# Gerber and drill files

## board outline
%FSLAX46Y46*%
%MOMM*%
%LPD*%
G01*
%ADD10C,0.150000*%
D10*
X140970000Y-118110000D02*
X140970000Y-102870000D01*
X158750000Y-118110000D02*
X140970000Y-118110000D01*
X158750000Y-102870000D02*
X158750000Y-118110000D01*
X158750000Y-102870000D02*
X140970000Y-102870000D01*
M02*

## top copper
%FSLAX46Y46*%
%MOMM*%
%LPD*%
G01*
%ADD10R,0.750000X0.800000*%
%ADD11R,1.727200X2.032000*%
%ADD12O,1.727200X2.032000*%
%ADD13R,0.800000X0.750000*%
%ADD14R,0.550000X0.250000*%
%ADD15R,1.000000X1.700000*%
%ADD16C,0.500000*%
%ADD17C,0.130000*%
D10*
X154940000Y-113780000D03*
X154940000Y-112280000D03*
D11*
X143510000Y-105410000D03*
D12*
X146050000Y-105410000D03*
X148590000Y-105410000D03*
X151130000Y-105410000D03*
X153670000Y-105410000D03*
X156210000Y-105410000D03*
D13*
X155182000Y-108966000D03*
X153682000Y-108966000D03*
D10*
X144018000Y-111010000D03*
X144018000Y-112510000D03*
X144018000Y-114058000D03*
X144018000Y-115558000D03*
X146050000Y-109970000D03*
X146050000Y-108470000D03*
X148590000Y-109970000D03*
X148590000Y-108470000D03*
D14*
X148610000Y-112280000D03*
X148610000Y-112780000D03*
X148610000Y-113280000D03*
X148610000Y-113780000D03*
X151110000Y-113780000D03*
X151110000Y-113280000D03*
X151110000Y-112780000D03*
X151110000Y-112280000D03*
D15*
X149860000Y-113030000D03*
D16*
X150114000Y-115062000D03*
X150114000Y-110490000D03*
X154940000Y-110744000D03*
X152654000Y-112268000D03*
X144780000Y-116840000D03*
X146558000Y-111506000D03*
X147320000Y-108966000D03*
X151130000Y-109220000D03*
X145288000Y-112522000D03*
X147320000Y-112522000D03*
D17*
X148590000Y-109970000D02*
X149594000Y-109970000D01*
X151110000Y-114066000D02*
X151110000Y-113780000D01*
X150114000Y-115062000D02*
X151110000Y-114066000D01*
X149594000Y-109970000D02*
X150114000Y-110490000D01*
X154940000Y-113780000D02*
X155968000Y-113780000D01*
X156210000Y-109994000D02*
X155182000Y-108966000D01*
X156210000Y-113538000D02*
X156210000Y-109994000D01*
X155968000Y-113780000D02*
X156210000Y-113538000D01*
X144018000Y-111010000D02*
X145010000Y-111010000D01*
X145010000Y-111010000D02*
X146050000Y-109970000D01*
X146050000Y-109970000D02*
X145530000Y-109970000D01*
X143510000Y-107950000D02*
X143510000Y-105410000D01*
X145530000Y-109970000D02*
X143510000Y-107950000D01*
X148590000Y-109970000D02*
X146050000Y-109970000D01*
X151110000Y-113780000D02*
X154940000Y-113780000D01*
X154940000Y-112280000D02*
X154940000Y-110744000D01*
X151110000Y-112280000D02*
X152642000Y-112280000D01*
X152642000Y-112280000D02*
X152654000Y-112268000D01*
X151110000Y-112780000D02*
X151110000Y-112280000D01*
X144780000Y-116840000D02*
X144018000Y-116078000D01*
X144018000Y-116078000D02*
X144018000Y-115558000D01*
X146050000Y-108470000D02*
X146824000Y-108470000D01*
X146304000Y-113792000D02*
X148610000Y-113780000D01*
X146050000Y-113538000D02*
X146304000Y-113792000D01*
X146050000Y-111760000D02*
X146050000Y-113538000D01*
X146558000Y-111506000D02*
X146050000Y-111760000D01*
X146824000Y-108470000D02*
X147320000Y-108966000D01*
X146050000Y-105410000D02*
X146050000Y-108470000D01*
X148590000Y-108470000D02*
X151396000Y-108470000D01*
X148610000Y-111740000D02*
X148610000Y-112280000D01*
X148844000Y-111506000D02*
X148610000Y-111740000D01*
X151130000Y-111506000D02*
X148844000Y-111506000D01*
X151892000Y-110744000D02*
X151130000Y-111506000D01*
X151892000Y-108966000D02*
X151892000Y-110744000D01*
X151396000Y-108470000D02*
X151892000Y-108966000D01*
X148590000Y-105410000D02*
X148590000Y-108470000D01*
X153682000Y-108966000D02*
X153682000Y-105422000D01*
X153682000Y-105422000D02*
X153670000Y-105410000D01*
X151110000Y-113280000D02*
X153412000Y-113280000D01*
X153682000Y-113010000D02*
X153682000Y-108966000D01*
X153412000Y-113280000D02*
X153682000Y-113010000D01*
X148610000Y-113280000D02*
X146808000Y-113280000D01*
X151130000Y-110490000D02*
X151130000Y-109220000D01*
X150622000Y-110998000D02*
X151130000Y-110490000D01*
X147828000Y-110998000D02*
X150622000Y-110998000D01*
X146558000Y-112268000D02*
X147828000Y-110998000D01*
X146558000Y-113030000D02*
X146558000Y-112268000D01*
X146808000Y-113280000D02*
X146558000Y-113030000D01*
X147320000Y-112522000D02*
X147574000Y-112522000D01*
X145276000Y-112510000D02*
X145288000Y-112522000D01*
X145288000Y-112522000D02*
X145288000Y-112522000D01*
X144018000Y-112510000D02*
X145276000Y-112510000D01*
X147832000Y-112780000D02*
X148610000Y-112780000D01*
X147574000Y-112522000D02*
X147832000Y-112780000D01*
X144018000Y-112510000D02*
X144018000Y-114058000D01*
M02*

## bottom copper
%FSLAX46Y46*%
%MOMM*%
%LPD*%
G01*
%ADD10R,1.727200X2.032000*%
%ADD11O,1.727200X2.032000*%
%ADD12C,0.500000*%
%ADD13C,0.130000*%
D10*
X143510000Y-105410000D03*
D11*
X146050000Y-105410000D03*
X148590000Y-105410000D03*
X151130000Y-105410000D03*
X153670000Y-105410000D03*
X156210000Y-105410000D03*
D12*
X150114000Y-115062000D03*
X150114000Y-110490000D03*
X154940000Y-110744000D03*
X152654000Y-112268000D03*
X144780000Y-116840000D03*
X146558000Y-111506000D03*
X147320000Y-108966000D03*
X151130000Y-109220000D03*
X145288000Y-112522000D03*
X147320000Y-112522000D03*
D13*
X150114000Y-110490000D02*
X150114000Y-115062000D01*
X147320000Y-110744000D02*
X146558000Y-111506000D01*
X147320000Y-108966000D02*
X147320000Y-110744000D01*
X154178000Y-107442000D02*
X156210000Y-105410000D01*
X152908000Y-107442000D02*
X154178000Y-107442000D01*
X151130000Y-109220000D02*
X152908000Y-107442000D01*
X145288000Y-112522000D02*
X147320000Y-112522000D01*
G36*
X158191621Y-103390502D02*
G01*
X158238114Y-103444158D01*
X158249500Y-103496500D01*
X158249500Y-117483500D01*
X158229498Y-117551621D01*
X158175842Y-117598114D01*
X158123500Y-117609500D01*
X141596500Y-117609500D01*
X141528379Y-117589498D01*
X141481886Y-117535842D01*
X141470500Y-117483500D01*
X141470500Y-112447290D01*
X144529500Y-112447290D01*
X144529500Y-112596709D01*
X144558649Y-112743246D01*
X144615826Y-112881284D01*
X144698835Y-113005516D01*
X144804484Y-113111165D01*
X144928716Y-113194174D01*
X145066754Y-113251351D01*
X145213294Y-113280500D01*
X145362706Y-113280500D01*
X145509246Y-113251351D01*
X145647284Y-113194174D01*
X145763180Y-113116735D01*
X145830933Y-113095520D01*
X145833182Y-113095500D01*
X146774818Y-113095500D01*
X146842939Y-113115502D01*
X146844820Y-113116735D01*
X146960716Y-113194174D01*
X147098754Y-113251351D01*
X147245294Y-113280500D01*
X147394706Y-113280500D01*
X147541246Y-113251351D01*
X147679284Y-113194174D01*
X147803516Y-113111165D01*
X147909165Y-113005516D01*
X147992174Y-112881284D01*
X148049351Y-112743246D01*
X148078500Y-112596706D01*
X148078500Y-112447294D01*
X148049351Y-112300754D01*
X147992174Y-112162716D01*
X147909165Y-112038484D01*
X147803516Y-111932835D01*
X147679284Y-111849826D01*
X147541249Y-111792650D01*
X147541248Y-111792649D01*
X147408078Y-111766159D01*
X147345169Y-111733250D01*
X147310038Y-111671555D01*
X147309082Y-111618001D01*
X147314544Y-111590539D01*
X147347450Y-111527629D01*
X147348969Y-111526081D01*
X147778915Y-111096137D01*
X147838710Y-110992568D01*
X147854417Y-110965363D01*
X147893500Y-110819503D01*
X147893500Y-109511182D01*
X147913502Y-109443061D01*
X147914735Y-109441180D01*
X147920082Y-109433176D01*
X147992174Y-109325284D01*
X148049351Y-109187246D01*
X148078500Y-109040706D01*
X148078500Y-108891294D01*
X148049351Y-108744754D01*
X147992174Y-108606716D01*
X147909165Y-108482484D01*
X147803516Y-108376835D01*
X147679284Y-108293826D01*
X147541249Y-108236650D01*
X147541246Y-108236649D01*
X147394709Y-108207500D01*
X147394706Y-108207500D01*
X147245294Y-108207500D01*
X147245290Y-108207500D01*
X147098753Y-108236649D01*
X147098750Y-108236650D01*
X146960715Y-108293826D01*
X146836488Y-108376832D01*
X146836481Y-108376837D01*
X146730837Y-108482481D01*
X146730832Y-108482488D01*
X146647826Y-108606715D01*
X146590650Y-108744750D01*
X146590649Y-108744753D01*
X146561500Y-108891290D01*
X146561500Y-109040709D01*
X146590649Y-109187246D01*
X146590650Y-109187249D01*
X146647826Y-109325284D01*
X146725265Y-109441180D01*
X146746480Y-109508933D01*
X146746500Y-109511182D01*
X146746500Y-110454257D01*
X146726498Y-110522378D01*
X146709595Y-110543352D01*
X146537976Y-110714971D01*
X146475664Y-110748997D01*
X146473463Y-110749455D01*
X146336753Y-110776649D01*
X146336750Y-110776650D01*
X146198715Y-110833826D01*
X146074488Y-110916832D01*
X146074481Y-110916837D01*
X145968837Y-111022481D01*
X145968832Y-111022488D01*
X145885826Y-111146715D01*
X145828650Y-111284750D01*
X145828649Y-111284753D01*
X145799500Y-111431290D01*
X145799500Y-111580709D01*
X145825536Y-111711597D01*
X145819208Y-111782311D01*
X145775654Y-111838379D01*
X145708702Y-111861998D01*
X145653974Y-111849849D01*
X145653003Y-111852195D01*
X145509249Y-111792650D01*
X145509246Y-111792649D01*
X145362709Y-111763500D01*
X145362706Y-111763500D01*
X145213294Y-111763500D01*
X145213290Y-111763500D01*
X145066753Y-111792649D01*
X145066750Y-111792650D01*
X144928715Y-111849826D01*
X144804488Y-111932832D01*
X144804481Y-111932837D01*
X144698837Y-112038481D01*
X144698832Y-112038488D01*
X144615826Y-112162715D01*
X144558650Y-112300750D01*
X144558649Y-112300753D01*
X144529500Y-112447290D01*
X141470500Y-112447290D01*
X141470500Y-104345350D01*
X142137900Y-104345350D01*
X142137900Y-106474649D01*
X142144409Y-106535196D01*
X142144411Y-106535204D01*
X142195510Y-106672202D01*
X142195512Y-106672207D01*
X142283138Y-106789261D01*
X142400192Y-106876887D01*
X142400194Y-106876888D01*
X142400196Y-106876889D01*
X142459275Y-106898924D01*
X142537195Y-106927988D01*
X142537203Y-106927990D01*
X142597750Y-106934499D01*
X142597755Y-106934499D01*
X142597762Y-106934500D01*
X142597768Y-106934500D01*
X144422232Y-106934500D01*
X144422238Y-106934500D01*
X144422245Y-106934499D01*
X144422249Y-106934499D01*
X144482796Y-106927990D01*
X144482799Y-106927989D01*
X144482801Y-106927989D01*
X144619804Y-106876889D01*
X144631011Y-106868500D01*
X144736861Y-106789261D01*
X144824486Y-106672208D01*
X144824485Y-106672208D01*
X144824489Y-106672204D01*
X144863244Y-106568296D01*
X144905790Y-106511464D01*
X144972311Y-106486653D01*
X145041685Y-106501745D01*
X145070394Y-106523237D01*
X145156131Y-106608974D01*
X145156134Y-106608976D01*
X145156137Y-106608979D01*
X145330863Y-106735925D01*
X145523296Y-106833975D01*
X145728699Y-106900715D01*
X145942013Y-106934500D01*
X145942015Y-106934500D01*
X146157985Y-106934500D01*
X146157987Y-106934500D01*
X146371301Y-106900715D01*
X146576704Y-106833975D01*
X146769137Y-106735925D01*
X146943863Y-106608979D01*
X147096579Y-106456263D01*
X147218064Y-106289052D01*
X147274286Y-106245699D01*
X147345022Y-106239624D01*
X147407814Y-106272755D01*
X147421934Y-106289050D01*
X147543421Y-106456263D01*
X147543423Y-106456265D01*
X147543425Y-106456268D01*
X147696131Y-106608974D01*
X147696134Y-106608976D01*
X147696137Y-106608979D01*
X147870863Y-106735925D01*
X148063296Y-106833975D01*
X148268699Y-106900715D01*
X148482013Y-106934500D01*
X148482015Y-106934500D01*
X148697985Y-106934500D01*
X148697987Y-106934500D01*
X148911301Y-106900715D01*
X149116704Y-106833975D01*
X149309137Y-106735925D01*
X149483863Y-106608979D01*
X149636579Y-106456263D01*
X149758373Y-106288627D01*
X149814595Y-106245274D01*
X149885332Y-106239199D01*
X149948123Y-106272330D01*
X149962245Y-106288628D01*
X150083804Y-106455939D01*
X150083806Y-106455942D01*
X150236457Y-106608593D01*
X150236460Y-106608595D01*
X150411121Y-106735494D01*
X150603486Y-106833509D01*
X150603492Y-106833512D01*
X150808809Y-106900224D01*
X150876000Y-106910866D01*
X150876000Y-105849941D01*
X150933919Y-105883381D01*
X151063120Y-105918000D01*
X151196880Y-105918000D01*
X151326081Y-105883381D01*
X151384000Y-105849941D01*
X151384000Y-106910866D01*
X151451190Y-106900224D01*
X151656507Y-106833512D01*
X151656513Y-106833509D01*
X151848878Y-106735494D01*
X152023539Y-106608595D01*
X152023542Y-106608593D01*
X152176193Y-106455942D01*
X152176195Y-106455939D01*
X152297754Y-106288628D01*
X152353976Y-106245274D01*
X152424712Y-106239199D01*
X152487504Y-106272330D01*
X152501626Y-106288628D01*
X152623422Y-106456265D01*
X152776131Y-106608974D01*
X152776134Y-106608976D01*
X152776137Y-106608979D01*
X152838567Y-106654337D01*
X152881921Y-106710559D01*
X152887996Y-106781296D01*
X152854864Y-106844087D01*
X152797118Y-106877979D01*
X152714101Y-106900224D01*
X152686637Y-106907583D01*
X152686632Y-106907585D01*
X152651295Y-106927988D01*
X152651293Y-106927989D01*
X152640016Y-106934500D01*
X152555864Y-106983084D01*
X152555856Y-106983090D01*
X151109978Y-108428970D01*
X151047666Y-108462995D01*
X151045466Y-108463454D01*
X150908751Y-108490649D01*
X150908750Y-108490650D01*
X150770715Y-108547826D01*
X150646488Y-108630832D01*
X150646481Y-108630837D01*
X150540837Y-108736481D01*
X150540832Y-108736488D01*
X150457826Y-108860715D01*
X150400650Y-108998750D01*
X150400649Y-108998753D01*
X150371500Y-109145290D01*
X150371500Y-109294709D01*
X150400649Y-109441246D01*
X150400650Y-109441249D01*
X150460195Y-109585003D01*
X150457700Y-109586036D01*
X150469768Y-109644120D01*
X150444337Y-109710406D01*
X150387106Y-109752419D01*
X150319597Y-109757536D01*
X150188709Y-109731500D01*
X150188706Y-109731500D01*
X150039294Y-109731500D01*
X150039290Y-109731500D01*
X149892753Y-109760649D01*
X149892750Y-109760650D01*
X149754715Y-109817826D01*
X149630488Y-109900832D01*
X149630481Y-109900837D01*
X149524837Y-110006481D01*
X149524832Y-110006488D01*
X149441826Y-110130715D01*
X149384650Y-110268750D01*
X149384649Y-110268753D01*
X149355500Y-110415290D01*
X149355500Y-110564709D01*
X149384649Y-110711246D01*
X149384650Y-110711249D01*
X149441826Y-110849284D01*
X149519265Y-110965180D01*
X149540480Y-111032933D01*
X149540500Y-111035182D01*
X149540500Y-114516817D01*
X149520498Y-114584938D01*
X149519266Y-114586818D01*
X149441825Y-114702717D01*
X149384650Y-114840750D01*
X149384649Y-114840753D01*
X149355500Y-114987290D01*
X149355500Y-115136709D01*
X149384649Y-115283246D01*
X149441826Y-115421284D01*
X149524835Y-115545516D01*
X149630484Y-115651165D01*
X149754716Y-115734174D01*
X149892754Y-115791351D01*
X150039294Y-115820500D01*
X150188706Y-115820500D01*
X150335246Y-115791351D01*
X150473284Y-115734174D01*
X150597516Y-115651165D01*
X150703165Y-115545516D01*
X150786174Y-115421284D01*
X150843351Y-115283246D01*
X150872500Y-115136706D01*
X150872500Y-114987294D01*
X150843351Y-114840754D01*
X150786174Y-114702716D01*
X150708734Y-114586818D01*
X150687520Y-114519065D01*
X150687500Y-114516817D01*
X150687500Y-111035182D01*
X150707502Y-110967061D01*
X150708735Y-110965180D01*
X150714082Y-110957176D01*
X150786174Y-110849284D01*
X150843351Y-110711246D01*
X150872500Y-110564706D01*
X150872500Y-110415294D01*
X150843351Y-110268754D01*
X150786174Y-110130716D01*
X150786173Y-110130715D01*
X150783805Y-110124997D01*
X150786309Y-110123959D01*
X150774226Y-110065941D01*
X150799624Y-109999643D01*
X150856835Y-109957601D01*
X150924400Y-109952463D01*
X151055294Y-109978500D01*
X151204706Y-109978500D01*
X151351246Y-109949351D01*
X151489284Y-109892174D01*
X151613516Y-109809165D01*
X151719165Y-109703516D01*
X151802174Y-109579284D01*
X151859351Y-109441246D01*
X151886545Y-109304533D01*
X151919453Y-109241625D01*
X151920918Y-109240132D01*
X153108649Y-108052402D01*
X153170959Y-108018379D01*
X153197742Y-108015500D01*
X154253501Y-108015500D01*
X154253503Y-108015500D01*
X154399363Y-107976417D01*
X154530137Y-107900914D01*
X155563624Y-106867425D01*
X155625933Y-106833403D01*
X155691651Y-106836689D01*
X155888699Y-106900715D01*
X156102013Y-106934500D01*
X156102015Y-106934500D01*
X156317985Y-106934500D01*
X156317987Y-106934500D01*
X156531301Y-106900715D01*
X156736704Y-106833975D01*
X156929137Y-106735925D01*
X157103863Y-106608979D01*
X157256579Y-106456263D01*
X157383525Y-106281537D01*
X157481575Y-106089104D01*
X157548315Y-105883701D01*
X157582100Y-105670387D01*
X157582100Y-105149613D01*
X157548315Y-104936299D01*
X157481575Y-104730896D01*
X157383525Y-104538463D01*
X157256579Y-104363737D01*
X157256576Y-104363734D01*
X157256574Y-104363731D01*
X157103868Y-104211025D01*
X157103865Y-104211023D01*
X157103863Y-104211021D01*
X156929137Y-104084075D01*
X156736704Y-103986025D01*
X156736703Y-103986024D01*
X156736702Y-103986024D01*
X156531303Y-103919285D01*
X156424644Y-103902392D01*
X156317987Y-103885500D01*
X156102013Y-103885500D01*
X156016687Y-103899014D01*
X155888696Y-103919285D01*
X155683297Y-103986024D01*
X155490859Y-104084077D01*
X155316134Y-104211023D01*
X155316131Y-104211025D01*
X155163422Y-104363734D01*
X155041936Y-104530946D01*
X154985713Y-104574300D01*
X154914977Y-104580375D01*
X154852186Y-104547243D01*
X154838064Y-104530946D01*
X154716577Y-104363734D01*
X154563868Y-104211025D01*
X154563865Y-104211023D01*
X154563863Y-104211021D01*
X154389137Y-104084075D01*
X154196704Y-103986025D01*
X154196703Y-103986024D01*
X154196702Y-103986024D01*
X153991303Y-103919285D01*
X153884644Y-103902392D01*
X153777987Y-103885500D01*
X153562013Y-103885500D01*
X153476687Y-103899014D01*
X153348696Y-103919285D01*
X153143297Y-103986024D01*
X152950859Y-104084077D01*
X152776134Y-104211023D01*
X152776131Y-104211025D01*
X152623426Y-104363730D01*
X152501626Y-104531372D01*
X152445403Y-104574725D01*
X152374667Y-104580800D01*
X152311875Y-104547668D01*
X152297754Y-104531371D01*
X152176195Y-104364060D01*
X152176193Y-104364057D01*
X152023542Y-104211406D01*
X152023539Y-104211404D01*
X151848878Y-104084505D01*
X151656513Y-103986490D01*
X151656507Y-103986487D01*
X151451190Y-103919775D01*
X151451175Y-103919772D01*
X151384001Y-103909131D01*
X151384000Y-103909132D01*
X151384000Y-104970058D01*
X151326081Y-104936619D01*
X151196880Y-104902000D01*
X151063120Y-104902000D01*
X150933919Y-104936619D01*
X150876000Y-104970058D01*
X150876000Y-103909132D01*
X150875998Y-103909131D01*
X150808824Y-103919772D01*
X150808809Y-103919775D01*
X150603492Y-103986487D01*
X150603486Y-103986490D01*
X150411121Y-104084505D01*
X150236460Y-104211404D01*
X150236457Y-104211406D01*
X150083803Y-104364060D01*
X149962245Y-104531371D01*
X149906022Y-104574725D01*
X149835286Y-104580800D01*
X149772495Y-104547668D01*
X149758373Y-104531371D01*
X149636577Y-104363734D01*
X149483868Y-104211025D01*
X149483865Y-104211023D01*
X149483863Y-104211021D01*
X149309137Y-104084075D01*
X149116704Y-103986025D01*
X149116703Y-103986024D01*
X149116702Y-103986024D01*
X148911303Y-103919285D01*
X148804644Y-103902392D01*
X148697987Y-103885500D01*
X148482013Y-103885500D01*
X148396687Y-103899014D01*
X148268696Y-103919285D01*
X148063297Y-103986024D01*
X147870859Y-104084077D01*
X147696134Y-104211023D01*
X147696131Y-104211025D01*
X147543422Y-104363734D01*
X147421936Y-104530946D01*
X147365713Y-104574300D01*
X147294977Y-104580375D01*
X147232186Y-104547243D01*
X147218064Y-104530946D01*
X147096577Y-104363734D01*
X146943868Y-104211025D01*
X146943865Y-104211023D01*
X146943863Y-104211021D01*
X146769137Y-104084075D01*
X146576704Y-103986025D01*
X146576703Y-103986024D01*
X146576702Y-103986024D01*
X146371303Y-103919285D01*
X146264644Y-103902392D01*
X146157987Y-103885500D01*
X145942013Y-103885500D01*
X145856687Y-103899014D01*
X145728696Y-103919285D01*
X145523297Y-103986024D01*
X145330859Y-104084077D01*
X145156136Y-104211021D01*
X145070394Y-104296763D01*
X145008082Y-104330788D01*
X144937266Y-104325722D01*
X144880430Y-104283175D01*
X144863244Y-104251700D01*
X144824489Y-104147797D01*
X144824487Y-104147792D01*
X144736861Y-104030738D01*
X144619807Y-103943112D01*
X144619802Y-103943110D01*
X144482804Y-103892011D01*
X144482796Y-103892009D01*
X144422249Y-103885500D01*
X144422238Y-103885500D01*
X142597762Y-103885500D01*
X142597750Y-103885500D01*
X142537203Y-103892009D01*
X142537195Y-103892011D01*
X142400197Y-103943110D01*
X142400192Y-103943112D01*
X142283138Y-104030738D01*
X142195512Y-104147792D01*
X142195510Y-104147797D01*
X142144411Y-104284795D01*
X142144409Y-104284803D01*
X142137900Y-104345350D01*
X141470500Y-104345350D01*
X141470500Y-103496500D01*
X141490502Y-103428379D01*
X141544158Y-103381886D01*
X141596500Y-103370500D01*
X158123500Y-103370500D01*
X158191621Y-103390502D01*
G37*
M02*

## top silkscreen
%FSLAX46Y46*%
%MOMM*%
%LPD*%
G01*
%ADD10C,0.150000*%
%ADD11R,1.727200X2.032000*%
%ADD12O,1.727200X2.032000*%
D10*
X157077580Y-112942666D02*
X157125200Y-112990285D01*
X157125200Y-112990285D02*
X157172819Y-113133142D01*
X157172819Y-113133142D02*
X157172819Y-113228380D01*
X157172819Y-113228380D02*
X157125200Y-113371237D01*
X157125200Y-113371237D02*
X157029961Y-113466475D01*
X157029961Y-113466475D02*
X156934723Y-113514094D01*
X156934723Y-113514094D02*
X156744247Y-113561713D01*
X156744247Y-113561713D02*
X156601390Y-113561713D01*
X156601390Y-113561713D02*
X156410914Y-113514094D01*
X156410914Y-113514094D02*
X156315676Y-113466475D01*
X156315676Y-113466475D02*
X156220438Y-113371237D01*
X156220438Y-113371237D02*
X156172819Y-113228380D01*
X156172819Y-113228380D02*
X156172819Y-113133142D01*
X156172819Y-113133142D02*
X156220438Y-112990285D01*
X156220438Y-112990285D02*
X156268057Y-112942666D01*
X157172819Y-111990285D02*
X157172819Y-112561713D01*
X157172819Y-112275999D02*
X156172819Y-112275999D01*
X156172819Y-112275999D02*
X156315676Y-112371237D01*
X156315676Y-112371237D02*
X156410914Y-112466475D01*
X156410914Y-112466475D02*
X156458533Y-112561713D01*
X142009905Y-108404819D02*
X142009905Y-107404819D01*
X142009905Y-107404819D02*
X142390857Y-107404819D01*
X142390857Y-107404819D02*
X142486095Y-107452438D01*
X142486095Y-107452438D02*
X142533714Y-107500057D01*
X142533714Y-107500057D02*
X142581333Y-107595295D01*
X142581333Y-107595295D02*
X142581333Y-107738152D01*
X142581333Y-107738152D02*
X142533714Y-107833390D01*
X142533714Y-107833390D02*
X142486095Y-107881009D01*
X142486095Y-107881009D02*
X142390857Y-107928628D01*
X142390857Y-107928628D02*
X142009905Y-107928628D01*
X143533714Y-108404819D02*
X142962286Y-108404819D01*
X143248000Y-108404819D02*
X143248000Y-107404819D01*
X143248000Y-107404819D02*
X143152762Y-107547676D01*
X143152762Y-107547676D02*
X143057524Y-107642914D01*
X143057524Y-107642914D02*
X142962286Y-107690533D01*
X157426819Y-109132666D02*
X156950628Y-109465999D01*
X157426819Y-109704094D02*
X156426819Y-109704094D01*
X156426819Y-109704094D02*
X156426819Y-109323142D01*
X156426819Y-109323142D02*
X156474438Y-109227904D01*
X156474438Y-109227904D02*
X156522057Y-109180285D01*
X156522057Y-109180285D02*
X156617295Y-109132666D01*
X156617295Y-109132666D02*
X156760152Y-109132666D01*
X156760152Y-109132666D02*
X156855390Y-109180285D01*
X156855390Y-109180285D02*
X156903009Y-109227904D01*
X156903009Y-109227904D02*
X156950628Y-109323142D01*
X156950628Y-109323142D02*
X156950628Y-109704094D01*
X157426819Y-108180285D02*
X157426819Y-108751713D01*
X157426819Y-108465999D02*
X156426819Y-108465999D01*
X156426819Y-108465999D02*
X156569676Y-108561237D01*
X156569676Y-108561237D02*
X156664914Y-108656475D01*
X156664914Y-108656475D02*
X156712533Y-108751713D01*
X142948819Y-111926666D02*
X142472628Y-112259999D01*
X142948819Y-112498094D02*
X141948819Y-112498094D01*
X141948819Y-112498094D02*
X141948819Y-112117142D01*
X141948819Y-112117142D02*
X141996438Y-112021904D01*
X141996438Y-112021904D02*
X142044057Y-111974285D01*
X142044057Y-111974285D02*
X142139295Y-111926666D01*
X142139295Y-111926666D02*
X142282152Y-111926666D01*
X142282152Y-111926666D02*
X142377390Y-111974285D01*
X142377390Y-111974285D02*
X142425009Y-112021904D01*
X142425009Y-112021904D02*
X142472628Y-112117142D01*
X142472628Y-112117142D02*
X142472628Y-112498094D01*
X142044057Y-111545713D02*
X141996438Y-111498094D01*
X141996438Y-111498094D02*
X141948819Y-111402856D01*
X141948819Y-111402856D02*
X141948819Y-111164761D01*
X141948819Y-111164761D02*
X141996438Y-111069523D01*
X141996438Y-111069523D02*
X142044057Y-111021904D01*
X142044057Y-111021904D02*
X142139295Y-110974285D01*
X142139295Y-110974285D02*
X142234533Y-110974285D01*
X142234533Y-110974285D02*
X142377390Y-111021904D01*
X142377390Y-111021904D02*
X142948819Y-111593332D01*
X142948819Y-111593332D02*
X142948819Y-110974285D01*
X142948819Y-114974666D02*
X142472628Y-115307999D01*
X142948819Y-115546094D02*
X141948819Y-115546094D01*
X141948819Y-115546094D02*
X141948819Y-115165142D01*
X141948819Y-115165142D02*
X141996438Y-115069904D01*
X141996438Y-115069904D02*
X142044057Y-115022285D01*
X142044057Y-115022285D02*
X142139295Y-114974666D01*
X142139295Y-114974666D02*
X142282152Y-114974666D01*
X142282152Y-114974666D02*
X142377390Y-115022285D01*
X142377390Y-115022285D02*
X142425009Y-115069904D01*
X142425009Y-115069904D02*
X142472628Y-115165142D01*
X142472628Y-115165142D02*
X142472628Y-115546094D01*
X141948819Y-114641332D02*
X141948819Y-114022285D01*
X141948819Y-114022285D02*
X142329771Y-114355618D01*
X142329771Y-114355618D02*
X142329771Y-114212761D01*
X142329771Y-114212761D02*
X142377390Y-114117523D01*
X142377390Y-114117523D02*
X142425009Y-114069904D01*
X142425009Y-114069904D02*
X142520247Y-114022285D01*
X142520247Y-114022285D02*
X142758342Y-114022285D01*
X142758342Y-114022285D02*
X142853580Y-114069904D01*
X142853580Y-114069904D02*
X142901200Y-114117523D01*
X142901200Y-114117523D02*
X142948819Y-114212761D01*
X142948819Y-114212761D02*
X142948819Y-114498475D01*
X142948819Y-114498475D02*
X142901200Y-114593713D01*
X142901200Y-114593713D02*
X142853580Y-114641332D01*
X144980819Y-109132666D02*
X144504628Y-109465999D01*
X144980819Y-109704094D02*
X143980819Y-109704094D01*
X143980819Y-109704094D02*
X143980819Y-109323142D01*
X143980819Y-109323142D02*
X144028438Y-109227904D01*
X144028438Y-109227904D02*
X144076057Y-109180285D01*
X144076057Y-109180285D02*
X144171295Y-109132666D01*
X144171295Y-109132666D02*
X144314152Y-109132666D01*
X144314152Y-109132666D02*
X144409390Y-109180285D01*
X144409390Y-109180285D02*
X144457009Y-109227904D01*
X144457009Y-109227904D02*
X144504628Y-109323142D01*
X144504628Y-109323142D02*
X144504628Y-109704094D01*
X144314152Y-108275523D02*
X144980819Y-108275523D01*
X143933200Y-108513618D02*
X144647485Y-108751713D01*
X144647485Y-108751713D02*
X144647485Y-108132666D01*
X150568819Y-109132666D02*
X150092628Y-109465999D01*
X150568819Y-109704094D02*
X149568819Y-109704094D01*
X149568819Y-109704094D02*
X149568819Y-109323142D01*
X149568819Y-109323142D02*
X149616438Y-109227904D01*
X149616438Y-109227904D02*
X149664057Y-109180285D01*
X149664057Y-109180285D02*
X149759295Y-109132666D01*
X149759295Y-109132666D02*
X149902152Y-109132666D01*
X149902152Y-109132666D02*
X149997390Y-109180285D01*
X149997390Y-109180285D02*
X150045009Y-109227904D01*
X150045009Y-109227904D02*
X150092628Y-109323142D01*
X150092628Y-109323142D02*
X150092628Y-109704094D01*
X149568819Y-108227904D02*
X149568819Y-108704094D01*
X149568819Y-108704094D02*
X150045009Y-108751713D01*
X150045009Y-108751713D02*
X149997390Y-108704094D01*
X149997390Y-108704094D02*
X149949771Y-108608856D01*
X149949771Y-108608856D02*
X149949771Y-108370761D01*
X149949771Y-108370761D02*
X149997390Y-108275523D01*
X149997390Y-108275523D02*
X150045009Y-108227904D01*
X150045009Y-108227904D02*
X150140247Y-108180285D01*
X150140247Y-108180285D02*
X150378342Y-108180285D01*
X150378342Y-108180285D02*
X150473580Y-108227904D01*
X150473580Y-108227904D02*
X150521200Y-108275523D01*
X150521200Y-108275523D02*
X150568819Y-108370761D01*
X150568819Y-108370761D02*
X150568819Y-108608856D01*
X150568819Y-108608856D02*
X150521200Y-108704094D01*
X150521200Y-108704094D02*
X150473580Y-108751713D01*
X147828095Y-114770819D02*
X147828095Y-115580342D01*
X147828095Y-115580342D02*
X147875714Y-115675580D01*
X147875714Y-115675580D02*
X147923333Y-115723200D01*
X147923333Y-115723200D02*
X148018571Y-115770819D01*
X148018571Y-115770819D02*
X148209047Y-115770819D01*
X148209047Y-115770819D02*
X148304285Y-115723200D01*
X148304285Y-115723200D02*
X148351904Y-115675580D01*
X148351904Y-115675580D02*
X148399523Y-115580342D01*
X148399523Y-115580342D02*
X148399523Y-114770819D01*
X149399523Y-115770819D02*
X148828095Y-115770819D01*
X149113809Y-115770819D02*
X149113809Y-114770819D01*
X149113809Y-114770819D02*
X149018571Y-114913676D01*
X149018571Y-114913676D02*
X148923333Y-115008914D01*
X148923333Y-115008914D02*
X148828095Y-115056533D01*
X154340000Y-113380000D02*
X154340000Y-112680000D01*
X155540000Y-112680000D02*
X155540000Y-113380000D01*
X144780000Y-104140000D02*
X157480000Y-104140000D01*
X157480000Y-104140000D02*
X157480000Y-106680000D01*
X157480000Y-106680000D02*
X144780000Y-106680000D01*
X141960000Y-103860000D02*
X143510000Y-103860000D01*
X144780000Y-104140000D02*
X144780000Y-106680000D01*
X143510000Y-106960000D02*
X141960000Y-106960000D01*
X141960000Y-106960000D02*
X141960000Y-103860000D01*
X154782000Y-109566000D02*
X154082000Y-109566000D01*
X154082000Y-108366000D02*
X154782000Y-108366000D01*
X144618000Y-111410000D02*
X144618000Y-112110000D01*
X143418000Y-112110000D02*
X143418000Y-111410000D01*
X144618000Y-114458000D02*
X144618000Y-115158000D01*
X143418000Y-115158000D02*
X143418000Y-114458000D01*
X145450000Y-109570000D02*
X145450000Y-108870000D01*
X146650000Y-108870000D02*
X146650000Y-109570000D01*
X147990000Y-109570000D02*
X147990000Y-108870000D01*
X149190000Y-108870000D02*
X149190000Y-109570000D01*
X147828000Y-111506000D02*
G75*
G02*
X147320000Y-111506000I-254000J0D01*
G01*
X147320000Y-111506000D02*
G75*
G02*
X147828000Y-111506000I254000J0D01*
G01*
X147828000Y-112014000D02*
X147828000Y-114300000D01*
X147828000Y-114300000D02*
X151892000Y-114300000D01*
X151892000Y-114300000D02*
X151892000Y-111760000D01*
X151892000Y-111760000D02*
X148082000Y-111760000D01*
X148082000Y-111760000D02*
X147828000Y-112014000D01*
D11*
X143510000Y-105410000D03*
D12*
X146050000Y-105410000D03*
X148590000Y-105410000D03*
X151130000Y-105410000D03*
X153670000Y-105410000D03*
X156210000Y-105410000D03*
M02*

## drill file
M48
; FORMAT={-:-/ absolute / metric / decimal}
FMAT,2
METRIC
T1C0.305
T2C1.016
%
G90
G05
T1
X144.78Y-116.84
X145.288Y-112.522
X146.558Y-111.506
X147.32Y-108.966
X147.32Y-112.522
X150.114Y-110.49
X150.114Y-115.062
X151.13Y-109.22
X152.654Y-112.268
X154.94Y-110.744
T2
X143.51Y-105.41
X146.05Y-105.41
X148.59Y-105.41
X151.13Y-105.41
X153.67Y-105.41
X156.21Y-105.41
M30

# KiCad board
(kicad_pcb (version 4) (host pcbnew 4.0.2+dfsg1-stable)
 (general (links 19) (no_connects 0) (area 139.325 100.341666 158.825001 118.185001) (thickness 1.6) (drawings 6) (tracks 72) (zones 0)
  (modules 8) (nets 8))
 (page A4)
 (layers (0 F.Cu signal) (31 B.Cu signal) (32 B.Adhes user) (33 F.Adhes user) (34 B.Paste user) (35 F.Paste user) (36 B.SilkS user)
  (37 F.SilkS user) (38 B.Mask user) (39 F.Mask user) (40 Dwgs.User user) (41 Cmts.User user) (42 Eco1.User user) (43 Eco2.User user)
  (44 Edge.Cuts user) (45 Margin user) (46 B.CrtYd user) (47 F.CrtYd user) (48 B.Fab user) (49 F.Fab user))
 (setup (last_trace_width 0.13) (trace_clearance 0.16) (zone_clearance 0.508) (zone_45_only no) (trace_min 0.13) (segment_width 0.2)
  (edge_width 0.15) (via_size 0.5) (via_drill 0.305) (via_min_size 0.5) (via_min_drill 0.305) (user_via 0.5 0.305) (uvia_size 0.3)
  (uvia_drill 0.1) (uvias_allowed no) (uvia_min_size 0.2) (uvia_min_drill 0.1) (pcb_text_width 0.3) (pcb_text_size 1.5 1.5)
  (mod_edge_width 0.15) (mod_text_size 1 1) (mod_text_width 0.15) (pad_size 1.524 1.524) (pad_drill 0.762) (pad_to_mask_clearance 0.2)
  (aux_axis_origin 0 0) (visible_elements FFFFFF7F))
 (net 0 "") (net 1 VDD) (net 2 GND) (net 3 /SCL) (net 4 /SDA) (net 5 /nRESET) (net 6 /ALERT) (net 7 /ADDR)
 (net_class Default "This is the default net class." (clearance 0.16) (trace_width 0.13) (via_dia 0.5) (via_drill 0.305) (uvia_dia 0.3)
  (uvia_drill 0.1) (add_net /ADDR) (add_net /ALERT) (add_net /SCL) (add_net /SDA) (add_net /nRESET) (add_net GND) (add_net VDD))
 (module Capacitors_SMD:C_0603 (layer F.Cu) (at 154.94 113.03 90)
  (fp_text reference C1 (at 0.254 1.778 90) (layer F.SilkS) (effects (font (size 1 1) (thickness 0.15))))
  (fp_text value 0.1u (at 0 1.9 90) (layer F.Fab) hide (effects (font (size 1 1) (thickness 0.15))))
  (fp_line (start -0.35 -0.6) (end 0.35 -0.6) (layer F.SilkS) (width 0.15))
  (fp_line (start 0.35 0.6) (end -0.35 0.6) (layer F.SilkS) (width 0.15))
  (pad 1 smd rect (at -0.75 0 90) (size 0.8 0.75) (layers F.Cu F.Paste F.Mask) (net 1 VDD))
  (pad 2 smd rect (at 0.75 0 90) (size 0.8 0.75) (layers F.Cu F.Paste F.Mask) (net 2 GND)))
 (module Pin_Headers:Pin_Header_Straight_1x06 (layer F.Cu) (at 143.51 105.41 90)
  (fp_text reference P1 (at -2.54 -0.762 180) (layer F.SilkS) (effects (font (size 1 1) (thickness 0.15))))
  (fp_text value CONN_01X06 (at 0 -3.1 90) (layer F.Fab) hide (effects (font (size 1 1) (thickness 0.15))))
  (fp_line (start 1.27 1.27) (end 1.27 13.97) (layer F.SilkS) (width 0.15))
  (fp_line (start 1.27 13.97) (end -1.27 13.97) (layer F.SilkS) (width 0.15))
  (fp_line (start -1.27 13.97) (end -1.27 1.27) (layer F.SilkS) (width 0.15))
  (fp_line (start 1.55 -1.55) (end 1.55 0) (layer F.SilkS) (width 0.15))
  (fp_line (start 1.27 1.27) (end -1.27 1.27) (layer F.SilkS) (width 0.15))
  (fp_line (start -1.55 0) (end -1.55 -1.55) (layer F.SilkS) (width 0.15))
  (fp_line (start -1.55 -1.55) (end 1.55 -1.55) (layer F.SilkS) (width 0.15))
  (pad 1 thru_hole rect (at 0 0 90) (size 2.032 1.7272) (drill 1.016) (layers *.Cu *.Mask F.SilkS) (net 1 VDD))
  (pad 2 thru_hole oval (at 0 2.54 90) (size 2.032 1.7272) (drill 1.016) (layers *.Cu *.Mask F.SilkS) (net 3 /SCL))
  (pad 3 thru_hole oval (at 0 5.08 90) (size 2.032 1.7272) (drill 1.016) (layers *.Cu *.Mask F.SilkS) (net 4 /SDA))
  (pad 4 thru_hole oval (at 0 7.62 90) (size 2.032 1.7272) (drill 1.016) (layers *.Cu *.Mask F.SilkS) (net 2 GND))
  (pad 5 thru_hole oval (at 0 10.16 90) (size 2.032 1.7272) (drill 1.016) (layers *.Cu *.Mask F.SilkS) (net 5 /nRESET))
  (pad 6 thru_hole oval (at 0 12.7 90) (size 2.032 1.7272) (drill 1.016) (layers *.Cu *.Mask F.SilkS) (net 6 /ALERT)))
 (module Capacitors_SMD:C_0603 (layer F.Cu) (at 154.432 108.966 180)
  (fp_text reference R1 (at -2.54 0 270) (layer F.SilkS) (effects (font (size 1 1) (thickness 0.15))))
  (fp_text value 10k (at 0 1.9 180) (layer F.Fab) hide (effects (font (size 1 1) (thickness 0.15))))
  (fp_line (start -0.35 -0.6) (end 0.35 -0.6) (layer F.SilkS) (width 0.15))
  (fp_line (start 0.35 0.6) (end -0.35 0.6) (layer F.SilkS) (width 0.15))
  (pad 1 smd rect (at -0.75 0 180) (size 0.8 0.75) (layers F.Cu F.Paste F.Mask) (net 1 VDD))
  (pad 2 smd rect (at 0.75 0 180) (size 0.8 0.75) (layers F.Cu F.Paste F.Mask) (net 5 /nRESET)))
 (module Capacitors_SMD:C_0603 (layer F.Cu) (at 144.018 111.76 270)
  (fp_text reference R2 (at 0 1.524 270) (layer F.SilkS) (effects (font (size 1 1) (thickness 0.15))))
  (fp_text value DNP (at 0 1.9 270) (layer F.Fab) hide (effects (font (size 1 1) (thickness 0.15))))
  (fp_line (start -0.35 -0.6) (end 0.35 -0.6) (layer F.SilkS) (width 0.15))
  (fp_line (start 0.35 0.6) (end -0.35 0.6) (layer F.SilkS) (width 0.15))
  (pad 1 smd rect (at -0.75 0 270) (size 0.8 0.75) (layers F.Cu F.Paste F.Mask) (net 1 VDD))
  (pad 2 smd rect (at 0.75 0 270) (size 0.8 0.75) (layers F.Cu F.Paste F.Mask) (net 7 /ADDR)))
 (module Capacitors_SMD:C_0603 (layer F.Cu) (at 144.018 114.808 270)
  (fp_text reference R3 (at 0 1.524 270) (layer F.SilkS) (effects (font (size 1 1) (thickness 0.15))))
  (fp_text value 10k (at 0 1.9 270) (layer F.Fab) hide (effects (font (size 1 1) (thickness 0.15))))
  (fp_line (start -0.35 -0.6) (end 0.35 -0.6) (layer F.SilkS) (width 0.15))
  (fp_line (start 0.35 0.6) (end -0.35 0.6) (layer F.SilkS) (width 0.15))
  (pad 1 smd rect (at -0.75 0 270) (size 0.8 0.75) (layers F.Cu F.Paste F.Mask) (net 7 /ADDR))
  (pad 2 smd rect (at 0.75 0 270) (size 0.8 0.75) (layers F.Cu F.Paste F.Mask) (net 2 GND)))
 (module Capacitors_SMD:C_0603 (layer F.Cu) (at 146.05 109.22 90)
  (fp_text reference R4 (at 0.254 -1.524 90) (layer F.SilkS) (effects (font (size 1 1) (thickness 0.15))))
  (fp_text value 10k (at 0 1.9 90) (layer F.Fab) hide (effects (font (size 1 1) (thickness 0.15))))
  (fp_line (start -0.35 -0.6) (end 0.35 -0.6) (layer F.SilkS) (width 0.15))
  (fp_line (start 0.35 0.6) (end -0.35 0.6) (layer F.SilkS) (width 0.15))
  (pad 1 smd rect (at -0.75 0 90) (size 0.8 0.75) (layers F.Cu F.Paste F.Mask) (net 1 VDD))
  (pad 2 smd rect (at 0.75 0 90) (size 0.8 0.75) (layers F.Cu F.Paste F.Mask) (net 3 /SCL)))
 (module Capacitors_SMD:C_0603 (layer F.Cu) (at 148.59 109.22 90)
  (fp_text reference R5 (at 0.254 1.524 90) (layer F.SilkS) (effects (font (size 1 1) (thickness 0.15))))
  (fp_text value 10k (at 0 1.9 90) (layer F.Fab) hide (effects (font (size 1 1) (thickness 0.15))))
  (fp_line (start -0.35 -0.6) (end 0.35 -0.6) (layer F.SilkS) (width 0.15))
  (fp_line (start 0.35 0.6) (end -0.35 0.6) (layer F.SilkS) (width 0.15))
  (pad 1 smd rect (at -0.75 0 90) (size 0.8 0.75) (layers F.Cu F.Paste F.Mask) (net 1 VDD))
  (pad 2 smd rect (at 0.75 0 90) (size 0.8 0.75) (layers F.Cu F.Paste F.Mask) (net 4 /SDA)))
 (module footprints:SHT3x (layer F.Cu) (at 149.86 113.03)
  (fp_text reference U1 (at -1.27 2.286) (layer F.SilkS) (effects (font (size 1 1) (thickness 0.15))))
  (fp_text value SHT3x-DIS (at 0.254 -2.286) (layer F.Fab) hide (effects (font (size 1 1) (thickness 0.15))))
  (fp_circle (center -2.286 -1.524) (end -2.032 -1.524) (layer F.SilkS) (width 0.15))
  (fp_line (start -2.032 -1.016) (end -2.032 1.27) (layer F.SilkS) (width 0.15))
  (fp_line (start -2.032 1.27) (end 2.032 1.27) (layer F.SilkS) (width 0.15))
  (fp_line (start 2.032 1.27) (end 2.032 -1.27) (layer F.SilkS) (width 0.15))
  (fp_line (start 2.032 -1.27) (end -1.778 -1.27) (layer F.SilkS) (width 0.15))
  (fp_line (start -1.778 -1.27) (end -2.032 -1.016) (layer F.SilkS) (width 0.15))
  (pad 1 smd rect (at -1.25 -0.75) (size 0.55 0.25) (layers F.Cu F.Paste F.Mask) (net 4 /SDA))
  (pad 2 smd rect (at -1.25 -0.25) (size 0.55 0.25) (layers F.Cu F.Paste F.Mask) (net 7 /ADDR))
  (pad 3 smd rect (at -1.25 0.25) (size 0.55 0.25) (layers F.Cu F.Paste F.Mask) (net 6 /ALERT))
  (pad 4 smd rect (at -1.25 0.75) (size 0.55 0.25) (layers F.Cu F.Paste F.Mask) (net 3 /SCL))
  (pad 5 smd rect (at 1.25 0.75) (size 0.55 0.25) (layers F.Cu F.Paste F.Mask) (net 1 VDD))
  (pad 6 smd rect (at 1.25 0.25) (size 0.55 0.25) (layers F.Cu F.Paste F.Mask) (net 5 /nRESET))
  (pad 7 smd rect (at 1.25 -0.25) (size 0.55 0.25) (layers F.Cu F.Paste F.Mask) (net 2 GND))
  (pad 8 smd rect (at 1.25 -0.75) (size 0.55 0.25) (layers F.Cu F.Paste F.Mask) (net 2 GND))
  (pad "" smd rect (at 0 0) (size 1 1.7) (layers F.Cu F.Paste F.Mask)))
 (gr_line (start 140.97 118.11) (end 140.97 102.87) (angle 90) (layer Edge.Cuts) (width 0.15))
 (gr_line (start 158.75 118.11) (end 140.97 118.11) (angle 90) (layer Edge.Cuts) (width 0.15))
 (gr_line (start 158.75 102.87) (end 158.75 118.11) (angle 90) (layer Edge.Cuts) (width 0.15))
 (gr_line (start 158.75 102.87) (end 140.97 102.87) (angle 90) (layer Edge.Cuts) (width 0.15))
 (segment (start 148.59 109.97) (end 149.594 109.97) (width 0.13) (layer F.Cu) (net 1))
 (segment (start 151.11 114.066) (end 151.11 113.78) (width 0.13) (layer F.Cu) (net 1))
 (segment (start 150.114 115.062) (end 151.11 114.066) (width 0.13) (layer F.Cu) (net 1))
 (via (at 150.114 115.062) (size 0.5) (drill 0.305) (layers F.Cu B.Cu) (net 1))
 (segment (start 150.114 110.49) (end 150.114 115.062) (width 0.13) (layer B.Cu) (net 1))
 (via (at 150.114 110.49) (size 0.5) (drill 0.305) (layers F.Cu B.Cu) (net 1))
 (segment (start 149.594 109.97) (end 150.114 110.49) (width 0.13) (layer F.Cu) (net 1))
 (segment (start 154.94 113.78) (end 155.968 113.78) (width 0.13) (layer F.Cu) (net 1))
 (segment (start 156.21 109.994) (end 155.182 108.966) (width 0.13) (layer F.Cu) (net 1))
 (segment (start 156.21 113.538) (end 156.21 109.994) (width 0.13) (layer F.Cu) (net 1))
 (segment (start 155.968 113.78) (end 156.21 113.538) (width 0.13) (layer F.Cu) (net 1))
 (segment (start 144.018 111.01) (end 145.01 111.01) (width 0.13) (layer F.Cu) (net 1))
 (segment (start 145.01 111.01) (end 146.05 109.97) (width 0.13) (layer F.Cu) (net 1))
 (segment (start 146.05 109.97) (end 145.53 109.97) (width 0.13) (layer F.Cu) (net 1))
 (segment (start 143.51 107.95) (end 143.51 105.41) (width 0.13) (layer F.Cu) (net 1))
 (segment (start 145.53 109.97) (end 143.51 107.95) (width 0.13) (layer F.Cu) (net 1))
 (segment (start 148.59 109.97) (end 146.05 109.97) (width 0.13) (layer F.Cu) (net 1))
 (segment (start 151.11 113.78) (end 154.94 113.78) (width 0.13) (layer F.Cu) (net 1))
 (segment (start 154.94 112.28) (end 154.94 110.744) (width 0.13) (layer F.Cu) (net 2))
 (via (at 154.94 110.744) (size 0.5) (drill 0.305) (layers F.Cu B.Cu) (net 2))
 (segment (start 151.11 112.28) (end 152.642 112.28) (width 0.13) (layer F.Cu) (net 2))
 (via (at 152.654 112.268) (size 0.5) (drill 0.305) (layers F.Cu B.Cu) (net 2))
 (segment (start 152.642 112.28) (end 152.654 112.268) (width 0.13) (layer F.Cu) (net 2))
 (segment (start 151.11 112.78) (end 151.11 112.28) (width 0.13) (layer F.Cu) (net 2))
 (via (at 144.78 116.84) (size 0.5) (drill 0.305) (layers F.Cu B.Cu) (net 2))
 (segment (start 144.78 116.84) (end 144.018 116.078) (width 0.13) (layer F.Cu) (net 2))
 (segment (start 144.018 116.078) (end 144.018 115.558) (width 0.13) (layer F.Cu) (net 2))
 (segment (start 146.05 108.47) (end 146.824 108.47) (width 0.13) (layer F.Cu) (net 3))
 (segment (start 146.304 113.792) (end 148.61 113.78) (width 0.13) (layer F.Cu) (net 3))
 (segment (start 146.05 113.538) (end 146.304 113.792) (width 0.13) (layer F.Cu) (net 3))
 (segment (start 146.05 111.76) (end 146.05 113.538) (width 0.13) (layer F.Cu) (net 3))
 (segment (start 146.558 111.506) (end 146.05 111.76) (width 0.13) (layer F.Cu) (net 3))
 (via (at 146.558 111.506) (size 0.5) (drill 0.305) (layers F.Cu B.Cu) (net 3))
 (segment (start 147.32 110.744) (end 146.558 111.506) (width 0.13) (layer B.Cu) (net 3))
 (segment (start 147.32 108.966) (end 147.32 110.744) (width 0.13) (layer B.Cu) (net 3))
 (via (at 147.32 108.966) (size 0.5) (drill 0.305) (layers F.Cu B.Cu) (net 3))
 (segment (start 146.824 108.47) (end 147.32 108.966) (width 0.13) (layer F.Cu) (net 3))
 (segment (start 146.05 105.41) (end 146.05 108.47) (width 0.13) (layer F.Cu) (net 3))
 (segment (start 148.59 108.47) (end 151.396 108.47) (width 0.13) (layer F.Cu) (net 4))
 (segment (start 148.61 111.74) (end 148.61 112.28) (width 0.13) (layer F.Cu) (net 4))
 (segment (start 148.844 111.506) (end 148.61 111.74) (width 0.13) (layer F.Cu) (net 4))
 (segment (start 151.13 111.506) (end 148.844 111.506) (width 0.13) (layer F.Cu) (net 4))
 (segment (start 151.892 110.744) (end 151.13 111.506) (width 0.13) (layer F.Cu) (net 4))
 (segment (start 151.892 108.966) (end 151.892 110.744) (width 0.13) (layer F.Cu) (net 4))
 (segment (start 151.396 108.47) (end 151.892 108.966) (width 0.13) (layer F.Cu) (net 4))
 (segment (start 148.59 105.41) (end 148.59 108.47) (width 0.13) (layer F.Cu) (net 4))
 (segment (start 153.682 108.966) (end 153.682 105.422) (width 0.13) (layer F.Cu) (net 5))
 (segment (start 153.682 105.422) (end 153.67 105.41) (width 0.13) (layer F.Cu) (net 5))
 (segment (start 151.11 113.28) (end 153.412 113.28) (width 0.13) (layer F.Cu) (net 5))
 (segment (start 153.682 113.01) (end 153.682 108.966) (width 0.13) (layer F.Cu) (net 5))
 (segment (start 153.412 113.28) (end 153.682 113.01) (width 0.13) (layer F.Cu) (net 5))
 (segment (start 148.61 113.28) (end 146.808 113.28) (width 0.13) (layer F.Cu) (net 6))
 (segment (start 154.178 107.442) (end 156.21 105.41) (width 0.13) (layer B.Cu) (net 6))
 (segment (start 152.908 107.442) (end 154.178 107.442) (width 0.13) (layer B.Cu) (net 6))
 (segment (start 151.13 109.22) (end 152.908 107.442) (width 0.13) (layer B.Cu) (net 6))
 (via (at 151.13 109.22) (size 0.5) (drill 0.305) (layers F.Cu B.Cu) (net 6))
 (segment (start 151.13 110.49) (end 151.13 109.22) (width 0.13) (layer F.Cu) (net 6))
 (segment (start 150.622 110.998) (end 151.13 110.49) (width 0.13) (layer F.Cu) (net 6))
 (segment (start 147.828 110.998) (end 150.622 110.998) (width 0.13) (layer F.Cu) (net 6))
 (segment (start 146.558 112.268) (end 147.828 110.998) (width 0.13) (layer F.Cu) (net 6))
 (segment (start 146.558 113.03) (end 146.558 112.268) (width 0.13) (layer F.Cu) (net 6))
 (segment (start 146.808 113.28) (end 146.558 113.03) (width 0.13) (layer F.Cu) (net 6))
 (segment (start 147.32 112.522) (end 147.574 112.522) (width 0.13) (layer F.Cu) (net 7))
 (segment (start 145.288 112.522) (end 147.32 112.522) (width 0.13) (layer B.Cu) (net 7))
 (segment (start 145.276 112.51) (end 145.288 112.522) (width 0.13) (layer F.Cu) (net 7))
 (segment (start 145.288 112.522) (end 145.288 112.522) (width 0.13) (layer F.Cu) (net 7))
 (via (at 145.288 112.522) (size 0.5) (drill 0.305) (layers F.Cu B.Cu) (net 7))
 (segment (start 144.018 112.51) (end 145.276 112.51) (width 0.13) (layer F.Cu) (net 7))
 (via (at 147.32 112.522) (size 0.5) (drill 0.305) (layers F.Cu B.Cu) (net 7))
 (segment (start 147.832 112.78) (end 148.61 112.78) (width 0.13) (layer F.Cu) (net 7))
 (segment (start 147.574 112.522) (end 147.832 112.78) (width 0.13) (layer F.Cu) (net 7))
 (segment (start 144.018 112.51) (end 144.018 114.058) (width 0.13) (layer F.Cu) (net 7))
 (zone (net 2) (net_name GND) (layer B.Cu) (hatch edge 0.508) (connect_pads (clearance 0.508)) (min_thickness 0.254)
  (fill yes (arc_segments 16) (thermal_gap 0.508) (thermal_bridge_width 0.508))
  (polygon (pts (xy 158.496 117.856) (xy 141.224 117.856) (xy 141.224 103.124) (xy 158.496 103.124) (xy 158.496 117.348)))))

